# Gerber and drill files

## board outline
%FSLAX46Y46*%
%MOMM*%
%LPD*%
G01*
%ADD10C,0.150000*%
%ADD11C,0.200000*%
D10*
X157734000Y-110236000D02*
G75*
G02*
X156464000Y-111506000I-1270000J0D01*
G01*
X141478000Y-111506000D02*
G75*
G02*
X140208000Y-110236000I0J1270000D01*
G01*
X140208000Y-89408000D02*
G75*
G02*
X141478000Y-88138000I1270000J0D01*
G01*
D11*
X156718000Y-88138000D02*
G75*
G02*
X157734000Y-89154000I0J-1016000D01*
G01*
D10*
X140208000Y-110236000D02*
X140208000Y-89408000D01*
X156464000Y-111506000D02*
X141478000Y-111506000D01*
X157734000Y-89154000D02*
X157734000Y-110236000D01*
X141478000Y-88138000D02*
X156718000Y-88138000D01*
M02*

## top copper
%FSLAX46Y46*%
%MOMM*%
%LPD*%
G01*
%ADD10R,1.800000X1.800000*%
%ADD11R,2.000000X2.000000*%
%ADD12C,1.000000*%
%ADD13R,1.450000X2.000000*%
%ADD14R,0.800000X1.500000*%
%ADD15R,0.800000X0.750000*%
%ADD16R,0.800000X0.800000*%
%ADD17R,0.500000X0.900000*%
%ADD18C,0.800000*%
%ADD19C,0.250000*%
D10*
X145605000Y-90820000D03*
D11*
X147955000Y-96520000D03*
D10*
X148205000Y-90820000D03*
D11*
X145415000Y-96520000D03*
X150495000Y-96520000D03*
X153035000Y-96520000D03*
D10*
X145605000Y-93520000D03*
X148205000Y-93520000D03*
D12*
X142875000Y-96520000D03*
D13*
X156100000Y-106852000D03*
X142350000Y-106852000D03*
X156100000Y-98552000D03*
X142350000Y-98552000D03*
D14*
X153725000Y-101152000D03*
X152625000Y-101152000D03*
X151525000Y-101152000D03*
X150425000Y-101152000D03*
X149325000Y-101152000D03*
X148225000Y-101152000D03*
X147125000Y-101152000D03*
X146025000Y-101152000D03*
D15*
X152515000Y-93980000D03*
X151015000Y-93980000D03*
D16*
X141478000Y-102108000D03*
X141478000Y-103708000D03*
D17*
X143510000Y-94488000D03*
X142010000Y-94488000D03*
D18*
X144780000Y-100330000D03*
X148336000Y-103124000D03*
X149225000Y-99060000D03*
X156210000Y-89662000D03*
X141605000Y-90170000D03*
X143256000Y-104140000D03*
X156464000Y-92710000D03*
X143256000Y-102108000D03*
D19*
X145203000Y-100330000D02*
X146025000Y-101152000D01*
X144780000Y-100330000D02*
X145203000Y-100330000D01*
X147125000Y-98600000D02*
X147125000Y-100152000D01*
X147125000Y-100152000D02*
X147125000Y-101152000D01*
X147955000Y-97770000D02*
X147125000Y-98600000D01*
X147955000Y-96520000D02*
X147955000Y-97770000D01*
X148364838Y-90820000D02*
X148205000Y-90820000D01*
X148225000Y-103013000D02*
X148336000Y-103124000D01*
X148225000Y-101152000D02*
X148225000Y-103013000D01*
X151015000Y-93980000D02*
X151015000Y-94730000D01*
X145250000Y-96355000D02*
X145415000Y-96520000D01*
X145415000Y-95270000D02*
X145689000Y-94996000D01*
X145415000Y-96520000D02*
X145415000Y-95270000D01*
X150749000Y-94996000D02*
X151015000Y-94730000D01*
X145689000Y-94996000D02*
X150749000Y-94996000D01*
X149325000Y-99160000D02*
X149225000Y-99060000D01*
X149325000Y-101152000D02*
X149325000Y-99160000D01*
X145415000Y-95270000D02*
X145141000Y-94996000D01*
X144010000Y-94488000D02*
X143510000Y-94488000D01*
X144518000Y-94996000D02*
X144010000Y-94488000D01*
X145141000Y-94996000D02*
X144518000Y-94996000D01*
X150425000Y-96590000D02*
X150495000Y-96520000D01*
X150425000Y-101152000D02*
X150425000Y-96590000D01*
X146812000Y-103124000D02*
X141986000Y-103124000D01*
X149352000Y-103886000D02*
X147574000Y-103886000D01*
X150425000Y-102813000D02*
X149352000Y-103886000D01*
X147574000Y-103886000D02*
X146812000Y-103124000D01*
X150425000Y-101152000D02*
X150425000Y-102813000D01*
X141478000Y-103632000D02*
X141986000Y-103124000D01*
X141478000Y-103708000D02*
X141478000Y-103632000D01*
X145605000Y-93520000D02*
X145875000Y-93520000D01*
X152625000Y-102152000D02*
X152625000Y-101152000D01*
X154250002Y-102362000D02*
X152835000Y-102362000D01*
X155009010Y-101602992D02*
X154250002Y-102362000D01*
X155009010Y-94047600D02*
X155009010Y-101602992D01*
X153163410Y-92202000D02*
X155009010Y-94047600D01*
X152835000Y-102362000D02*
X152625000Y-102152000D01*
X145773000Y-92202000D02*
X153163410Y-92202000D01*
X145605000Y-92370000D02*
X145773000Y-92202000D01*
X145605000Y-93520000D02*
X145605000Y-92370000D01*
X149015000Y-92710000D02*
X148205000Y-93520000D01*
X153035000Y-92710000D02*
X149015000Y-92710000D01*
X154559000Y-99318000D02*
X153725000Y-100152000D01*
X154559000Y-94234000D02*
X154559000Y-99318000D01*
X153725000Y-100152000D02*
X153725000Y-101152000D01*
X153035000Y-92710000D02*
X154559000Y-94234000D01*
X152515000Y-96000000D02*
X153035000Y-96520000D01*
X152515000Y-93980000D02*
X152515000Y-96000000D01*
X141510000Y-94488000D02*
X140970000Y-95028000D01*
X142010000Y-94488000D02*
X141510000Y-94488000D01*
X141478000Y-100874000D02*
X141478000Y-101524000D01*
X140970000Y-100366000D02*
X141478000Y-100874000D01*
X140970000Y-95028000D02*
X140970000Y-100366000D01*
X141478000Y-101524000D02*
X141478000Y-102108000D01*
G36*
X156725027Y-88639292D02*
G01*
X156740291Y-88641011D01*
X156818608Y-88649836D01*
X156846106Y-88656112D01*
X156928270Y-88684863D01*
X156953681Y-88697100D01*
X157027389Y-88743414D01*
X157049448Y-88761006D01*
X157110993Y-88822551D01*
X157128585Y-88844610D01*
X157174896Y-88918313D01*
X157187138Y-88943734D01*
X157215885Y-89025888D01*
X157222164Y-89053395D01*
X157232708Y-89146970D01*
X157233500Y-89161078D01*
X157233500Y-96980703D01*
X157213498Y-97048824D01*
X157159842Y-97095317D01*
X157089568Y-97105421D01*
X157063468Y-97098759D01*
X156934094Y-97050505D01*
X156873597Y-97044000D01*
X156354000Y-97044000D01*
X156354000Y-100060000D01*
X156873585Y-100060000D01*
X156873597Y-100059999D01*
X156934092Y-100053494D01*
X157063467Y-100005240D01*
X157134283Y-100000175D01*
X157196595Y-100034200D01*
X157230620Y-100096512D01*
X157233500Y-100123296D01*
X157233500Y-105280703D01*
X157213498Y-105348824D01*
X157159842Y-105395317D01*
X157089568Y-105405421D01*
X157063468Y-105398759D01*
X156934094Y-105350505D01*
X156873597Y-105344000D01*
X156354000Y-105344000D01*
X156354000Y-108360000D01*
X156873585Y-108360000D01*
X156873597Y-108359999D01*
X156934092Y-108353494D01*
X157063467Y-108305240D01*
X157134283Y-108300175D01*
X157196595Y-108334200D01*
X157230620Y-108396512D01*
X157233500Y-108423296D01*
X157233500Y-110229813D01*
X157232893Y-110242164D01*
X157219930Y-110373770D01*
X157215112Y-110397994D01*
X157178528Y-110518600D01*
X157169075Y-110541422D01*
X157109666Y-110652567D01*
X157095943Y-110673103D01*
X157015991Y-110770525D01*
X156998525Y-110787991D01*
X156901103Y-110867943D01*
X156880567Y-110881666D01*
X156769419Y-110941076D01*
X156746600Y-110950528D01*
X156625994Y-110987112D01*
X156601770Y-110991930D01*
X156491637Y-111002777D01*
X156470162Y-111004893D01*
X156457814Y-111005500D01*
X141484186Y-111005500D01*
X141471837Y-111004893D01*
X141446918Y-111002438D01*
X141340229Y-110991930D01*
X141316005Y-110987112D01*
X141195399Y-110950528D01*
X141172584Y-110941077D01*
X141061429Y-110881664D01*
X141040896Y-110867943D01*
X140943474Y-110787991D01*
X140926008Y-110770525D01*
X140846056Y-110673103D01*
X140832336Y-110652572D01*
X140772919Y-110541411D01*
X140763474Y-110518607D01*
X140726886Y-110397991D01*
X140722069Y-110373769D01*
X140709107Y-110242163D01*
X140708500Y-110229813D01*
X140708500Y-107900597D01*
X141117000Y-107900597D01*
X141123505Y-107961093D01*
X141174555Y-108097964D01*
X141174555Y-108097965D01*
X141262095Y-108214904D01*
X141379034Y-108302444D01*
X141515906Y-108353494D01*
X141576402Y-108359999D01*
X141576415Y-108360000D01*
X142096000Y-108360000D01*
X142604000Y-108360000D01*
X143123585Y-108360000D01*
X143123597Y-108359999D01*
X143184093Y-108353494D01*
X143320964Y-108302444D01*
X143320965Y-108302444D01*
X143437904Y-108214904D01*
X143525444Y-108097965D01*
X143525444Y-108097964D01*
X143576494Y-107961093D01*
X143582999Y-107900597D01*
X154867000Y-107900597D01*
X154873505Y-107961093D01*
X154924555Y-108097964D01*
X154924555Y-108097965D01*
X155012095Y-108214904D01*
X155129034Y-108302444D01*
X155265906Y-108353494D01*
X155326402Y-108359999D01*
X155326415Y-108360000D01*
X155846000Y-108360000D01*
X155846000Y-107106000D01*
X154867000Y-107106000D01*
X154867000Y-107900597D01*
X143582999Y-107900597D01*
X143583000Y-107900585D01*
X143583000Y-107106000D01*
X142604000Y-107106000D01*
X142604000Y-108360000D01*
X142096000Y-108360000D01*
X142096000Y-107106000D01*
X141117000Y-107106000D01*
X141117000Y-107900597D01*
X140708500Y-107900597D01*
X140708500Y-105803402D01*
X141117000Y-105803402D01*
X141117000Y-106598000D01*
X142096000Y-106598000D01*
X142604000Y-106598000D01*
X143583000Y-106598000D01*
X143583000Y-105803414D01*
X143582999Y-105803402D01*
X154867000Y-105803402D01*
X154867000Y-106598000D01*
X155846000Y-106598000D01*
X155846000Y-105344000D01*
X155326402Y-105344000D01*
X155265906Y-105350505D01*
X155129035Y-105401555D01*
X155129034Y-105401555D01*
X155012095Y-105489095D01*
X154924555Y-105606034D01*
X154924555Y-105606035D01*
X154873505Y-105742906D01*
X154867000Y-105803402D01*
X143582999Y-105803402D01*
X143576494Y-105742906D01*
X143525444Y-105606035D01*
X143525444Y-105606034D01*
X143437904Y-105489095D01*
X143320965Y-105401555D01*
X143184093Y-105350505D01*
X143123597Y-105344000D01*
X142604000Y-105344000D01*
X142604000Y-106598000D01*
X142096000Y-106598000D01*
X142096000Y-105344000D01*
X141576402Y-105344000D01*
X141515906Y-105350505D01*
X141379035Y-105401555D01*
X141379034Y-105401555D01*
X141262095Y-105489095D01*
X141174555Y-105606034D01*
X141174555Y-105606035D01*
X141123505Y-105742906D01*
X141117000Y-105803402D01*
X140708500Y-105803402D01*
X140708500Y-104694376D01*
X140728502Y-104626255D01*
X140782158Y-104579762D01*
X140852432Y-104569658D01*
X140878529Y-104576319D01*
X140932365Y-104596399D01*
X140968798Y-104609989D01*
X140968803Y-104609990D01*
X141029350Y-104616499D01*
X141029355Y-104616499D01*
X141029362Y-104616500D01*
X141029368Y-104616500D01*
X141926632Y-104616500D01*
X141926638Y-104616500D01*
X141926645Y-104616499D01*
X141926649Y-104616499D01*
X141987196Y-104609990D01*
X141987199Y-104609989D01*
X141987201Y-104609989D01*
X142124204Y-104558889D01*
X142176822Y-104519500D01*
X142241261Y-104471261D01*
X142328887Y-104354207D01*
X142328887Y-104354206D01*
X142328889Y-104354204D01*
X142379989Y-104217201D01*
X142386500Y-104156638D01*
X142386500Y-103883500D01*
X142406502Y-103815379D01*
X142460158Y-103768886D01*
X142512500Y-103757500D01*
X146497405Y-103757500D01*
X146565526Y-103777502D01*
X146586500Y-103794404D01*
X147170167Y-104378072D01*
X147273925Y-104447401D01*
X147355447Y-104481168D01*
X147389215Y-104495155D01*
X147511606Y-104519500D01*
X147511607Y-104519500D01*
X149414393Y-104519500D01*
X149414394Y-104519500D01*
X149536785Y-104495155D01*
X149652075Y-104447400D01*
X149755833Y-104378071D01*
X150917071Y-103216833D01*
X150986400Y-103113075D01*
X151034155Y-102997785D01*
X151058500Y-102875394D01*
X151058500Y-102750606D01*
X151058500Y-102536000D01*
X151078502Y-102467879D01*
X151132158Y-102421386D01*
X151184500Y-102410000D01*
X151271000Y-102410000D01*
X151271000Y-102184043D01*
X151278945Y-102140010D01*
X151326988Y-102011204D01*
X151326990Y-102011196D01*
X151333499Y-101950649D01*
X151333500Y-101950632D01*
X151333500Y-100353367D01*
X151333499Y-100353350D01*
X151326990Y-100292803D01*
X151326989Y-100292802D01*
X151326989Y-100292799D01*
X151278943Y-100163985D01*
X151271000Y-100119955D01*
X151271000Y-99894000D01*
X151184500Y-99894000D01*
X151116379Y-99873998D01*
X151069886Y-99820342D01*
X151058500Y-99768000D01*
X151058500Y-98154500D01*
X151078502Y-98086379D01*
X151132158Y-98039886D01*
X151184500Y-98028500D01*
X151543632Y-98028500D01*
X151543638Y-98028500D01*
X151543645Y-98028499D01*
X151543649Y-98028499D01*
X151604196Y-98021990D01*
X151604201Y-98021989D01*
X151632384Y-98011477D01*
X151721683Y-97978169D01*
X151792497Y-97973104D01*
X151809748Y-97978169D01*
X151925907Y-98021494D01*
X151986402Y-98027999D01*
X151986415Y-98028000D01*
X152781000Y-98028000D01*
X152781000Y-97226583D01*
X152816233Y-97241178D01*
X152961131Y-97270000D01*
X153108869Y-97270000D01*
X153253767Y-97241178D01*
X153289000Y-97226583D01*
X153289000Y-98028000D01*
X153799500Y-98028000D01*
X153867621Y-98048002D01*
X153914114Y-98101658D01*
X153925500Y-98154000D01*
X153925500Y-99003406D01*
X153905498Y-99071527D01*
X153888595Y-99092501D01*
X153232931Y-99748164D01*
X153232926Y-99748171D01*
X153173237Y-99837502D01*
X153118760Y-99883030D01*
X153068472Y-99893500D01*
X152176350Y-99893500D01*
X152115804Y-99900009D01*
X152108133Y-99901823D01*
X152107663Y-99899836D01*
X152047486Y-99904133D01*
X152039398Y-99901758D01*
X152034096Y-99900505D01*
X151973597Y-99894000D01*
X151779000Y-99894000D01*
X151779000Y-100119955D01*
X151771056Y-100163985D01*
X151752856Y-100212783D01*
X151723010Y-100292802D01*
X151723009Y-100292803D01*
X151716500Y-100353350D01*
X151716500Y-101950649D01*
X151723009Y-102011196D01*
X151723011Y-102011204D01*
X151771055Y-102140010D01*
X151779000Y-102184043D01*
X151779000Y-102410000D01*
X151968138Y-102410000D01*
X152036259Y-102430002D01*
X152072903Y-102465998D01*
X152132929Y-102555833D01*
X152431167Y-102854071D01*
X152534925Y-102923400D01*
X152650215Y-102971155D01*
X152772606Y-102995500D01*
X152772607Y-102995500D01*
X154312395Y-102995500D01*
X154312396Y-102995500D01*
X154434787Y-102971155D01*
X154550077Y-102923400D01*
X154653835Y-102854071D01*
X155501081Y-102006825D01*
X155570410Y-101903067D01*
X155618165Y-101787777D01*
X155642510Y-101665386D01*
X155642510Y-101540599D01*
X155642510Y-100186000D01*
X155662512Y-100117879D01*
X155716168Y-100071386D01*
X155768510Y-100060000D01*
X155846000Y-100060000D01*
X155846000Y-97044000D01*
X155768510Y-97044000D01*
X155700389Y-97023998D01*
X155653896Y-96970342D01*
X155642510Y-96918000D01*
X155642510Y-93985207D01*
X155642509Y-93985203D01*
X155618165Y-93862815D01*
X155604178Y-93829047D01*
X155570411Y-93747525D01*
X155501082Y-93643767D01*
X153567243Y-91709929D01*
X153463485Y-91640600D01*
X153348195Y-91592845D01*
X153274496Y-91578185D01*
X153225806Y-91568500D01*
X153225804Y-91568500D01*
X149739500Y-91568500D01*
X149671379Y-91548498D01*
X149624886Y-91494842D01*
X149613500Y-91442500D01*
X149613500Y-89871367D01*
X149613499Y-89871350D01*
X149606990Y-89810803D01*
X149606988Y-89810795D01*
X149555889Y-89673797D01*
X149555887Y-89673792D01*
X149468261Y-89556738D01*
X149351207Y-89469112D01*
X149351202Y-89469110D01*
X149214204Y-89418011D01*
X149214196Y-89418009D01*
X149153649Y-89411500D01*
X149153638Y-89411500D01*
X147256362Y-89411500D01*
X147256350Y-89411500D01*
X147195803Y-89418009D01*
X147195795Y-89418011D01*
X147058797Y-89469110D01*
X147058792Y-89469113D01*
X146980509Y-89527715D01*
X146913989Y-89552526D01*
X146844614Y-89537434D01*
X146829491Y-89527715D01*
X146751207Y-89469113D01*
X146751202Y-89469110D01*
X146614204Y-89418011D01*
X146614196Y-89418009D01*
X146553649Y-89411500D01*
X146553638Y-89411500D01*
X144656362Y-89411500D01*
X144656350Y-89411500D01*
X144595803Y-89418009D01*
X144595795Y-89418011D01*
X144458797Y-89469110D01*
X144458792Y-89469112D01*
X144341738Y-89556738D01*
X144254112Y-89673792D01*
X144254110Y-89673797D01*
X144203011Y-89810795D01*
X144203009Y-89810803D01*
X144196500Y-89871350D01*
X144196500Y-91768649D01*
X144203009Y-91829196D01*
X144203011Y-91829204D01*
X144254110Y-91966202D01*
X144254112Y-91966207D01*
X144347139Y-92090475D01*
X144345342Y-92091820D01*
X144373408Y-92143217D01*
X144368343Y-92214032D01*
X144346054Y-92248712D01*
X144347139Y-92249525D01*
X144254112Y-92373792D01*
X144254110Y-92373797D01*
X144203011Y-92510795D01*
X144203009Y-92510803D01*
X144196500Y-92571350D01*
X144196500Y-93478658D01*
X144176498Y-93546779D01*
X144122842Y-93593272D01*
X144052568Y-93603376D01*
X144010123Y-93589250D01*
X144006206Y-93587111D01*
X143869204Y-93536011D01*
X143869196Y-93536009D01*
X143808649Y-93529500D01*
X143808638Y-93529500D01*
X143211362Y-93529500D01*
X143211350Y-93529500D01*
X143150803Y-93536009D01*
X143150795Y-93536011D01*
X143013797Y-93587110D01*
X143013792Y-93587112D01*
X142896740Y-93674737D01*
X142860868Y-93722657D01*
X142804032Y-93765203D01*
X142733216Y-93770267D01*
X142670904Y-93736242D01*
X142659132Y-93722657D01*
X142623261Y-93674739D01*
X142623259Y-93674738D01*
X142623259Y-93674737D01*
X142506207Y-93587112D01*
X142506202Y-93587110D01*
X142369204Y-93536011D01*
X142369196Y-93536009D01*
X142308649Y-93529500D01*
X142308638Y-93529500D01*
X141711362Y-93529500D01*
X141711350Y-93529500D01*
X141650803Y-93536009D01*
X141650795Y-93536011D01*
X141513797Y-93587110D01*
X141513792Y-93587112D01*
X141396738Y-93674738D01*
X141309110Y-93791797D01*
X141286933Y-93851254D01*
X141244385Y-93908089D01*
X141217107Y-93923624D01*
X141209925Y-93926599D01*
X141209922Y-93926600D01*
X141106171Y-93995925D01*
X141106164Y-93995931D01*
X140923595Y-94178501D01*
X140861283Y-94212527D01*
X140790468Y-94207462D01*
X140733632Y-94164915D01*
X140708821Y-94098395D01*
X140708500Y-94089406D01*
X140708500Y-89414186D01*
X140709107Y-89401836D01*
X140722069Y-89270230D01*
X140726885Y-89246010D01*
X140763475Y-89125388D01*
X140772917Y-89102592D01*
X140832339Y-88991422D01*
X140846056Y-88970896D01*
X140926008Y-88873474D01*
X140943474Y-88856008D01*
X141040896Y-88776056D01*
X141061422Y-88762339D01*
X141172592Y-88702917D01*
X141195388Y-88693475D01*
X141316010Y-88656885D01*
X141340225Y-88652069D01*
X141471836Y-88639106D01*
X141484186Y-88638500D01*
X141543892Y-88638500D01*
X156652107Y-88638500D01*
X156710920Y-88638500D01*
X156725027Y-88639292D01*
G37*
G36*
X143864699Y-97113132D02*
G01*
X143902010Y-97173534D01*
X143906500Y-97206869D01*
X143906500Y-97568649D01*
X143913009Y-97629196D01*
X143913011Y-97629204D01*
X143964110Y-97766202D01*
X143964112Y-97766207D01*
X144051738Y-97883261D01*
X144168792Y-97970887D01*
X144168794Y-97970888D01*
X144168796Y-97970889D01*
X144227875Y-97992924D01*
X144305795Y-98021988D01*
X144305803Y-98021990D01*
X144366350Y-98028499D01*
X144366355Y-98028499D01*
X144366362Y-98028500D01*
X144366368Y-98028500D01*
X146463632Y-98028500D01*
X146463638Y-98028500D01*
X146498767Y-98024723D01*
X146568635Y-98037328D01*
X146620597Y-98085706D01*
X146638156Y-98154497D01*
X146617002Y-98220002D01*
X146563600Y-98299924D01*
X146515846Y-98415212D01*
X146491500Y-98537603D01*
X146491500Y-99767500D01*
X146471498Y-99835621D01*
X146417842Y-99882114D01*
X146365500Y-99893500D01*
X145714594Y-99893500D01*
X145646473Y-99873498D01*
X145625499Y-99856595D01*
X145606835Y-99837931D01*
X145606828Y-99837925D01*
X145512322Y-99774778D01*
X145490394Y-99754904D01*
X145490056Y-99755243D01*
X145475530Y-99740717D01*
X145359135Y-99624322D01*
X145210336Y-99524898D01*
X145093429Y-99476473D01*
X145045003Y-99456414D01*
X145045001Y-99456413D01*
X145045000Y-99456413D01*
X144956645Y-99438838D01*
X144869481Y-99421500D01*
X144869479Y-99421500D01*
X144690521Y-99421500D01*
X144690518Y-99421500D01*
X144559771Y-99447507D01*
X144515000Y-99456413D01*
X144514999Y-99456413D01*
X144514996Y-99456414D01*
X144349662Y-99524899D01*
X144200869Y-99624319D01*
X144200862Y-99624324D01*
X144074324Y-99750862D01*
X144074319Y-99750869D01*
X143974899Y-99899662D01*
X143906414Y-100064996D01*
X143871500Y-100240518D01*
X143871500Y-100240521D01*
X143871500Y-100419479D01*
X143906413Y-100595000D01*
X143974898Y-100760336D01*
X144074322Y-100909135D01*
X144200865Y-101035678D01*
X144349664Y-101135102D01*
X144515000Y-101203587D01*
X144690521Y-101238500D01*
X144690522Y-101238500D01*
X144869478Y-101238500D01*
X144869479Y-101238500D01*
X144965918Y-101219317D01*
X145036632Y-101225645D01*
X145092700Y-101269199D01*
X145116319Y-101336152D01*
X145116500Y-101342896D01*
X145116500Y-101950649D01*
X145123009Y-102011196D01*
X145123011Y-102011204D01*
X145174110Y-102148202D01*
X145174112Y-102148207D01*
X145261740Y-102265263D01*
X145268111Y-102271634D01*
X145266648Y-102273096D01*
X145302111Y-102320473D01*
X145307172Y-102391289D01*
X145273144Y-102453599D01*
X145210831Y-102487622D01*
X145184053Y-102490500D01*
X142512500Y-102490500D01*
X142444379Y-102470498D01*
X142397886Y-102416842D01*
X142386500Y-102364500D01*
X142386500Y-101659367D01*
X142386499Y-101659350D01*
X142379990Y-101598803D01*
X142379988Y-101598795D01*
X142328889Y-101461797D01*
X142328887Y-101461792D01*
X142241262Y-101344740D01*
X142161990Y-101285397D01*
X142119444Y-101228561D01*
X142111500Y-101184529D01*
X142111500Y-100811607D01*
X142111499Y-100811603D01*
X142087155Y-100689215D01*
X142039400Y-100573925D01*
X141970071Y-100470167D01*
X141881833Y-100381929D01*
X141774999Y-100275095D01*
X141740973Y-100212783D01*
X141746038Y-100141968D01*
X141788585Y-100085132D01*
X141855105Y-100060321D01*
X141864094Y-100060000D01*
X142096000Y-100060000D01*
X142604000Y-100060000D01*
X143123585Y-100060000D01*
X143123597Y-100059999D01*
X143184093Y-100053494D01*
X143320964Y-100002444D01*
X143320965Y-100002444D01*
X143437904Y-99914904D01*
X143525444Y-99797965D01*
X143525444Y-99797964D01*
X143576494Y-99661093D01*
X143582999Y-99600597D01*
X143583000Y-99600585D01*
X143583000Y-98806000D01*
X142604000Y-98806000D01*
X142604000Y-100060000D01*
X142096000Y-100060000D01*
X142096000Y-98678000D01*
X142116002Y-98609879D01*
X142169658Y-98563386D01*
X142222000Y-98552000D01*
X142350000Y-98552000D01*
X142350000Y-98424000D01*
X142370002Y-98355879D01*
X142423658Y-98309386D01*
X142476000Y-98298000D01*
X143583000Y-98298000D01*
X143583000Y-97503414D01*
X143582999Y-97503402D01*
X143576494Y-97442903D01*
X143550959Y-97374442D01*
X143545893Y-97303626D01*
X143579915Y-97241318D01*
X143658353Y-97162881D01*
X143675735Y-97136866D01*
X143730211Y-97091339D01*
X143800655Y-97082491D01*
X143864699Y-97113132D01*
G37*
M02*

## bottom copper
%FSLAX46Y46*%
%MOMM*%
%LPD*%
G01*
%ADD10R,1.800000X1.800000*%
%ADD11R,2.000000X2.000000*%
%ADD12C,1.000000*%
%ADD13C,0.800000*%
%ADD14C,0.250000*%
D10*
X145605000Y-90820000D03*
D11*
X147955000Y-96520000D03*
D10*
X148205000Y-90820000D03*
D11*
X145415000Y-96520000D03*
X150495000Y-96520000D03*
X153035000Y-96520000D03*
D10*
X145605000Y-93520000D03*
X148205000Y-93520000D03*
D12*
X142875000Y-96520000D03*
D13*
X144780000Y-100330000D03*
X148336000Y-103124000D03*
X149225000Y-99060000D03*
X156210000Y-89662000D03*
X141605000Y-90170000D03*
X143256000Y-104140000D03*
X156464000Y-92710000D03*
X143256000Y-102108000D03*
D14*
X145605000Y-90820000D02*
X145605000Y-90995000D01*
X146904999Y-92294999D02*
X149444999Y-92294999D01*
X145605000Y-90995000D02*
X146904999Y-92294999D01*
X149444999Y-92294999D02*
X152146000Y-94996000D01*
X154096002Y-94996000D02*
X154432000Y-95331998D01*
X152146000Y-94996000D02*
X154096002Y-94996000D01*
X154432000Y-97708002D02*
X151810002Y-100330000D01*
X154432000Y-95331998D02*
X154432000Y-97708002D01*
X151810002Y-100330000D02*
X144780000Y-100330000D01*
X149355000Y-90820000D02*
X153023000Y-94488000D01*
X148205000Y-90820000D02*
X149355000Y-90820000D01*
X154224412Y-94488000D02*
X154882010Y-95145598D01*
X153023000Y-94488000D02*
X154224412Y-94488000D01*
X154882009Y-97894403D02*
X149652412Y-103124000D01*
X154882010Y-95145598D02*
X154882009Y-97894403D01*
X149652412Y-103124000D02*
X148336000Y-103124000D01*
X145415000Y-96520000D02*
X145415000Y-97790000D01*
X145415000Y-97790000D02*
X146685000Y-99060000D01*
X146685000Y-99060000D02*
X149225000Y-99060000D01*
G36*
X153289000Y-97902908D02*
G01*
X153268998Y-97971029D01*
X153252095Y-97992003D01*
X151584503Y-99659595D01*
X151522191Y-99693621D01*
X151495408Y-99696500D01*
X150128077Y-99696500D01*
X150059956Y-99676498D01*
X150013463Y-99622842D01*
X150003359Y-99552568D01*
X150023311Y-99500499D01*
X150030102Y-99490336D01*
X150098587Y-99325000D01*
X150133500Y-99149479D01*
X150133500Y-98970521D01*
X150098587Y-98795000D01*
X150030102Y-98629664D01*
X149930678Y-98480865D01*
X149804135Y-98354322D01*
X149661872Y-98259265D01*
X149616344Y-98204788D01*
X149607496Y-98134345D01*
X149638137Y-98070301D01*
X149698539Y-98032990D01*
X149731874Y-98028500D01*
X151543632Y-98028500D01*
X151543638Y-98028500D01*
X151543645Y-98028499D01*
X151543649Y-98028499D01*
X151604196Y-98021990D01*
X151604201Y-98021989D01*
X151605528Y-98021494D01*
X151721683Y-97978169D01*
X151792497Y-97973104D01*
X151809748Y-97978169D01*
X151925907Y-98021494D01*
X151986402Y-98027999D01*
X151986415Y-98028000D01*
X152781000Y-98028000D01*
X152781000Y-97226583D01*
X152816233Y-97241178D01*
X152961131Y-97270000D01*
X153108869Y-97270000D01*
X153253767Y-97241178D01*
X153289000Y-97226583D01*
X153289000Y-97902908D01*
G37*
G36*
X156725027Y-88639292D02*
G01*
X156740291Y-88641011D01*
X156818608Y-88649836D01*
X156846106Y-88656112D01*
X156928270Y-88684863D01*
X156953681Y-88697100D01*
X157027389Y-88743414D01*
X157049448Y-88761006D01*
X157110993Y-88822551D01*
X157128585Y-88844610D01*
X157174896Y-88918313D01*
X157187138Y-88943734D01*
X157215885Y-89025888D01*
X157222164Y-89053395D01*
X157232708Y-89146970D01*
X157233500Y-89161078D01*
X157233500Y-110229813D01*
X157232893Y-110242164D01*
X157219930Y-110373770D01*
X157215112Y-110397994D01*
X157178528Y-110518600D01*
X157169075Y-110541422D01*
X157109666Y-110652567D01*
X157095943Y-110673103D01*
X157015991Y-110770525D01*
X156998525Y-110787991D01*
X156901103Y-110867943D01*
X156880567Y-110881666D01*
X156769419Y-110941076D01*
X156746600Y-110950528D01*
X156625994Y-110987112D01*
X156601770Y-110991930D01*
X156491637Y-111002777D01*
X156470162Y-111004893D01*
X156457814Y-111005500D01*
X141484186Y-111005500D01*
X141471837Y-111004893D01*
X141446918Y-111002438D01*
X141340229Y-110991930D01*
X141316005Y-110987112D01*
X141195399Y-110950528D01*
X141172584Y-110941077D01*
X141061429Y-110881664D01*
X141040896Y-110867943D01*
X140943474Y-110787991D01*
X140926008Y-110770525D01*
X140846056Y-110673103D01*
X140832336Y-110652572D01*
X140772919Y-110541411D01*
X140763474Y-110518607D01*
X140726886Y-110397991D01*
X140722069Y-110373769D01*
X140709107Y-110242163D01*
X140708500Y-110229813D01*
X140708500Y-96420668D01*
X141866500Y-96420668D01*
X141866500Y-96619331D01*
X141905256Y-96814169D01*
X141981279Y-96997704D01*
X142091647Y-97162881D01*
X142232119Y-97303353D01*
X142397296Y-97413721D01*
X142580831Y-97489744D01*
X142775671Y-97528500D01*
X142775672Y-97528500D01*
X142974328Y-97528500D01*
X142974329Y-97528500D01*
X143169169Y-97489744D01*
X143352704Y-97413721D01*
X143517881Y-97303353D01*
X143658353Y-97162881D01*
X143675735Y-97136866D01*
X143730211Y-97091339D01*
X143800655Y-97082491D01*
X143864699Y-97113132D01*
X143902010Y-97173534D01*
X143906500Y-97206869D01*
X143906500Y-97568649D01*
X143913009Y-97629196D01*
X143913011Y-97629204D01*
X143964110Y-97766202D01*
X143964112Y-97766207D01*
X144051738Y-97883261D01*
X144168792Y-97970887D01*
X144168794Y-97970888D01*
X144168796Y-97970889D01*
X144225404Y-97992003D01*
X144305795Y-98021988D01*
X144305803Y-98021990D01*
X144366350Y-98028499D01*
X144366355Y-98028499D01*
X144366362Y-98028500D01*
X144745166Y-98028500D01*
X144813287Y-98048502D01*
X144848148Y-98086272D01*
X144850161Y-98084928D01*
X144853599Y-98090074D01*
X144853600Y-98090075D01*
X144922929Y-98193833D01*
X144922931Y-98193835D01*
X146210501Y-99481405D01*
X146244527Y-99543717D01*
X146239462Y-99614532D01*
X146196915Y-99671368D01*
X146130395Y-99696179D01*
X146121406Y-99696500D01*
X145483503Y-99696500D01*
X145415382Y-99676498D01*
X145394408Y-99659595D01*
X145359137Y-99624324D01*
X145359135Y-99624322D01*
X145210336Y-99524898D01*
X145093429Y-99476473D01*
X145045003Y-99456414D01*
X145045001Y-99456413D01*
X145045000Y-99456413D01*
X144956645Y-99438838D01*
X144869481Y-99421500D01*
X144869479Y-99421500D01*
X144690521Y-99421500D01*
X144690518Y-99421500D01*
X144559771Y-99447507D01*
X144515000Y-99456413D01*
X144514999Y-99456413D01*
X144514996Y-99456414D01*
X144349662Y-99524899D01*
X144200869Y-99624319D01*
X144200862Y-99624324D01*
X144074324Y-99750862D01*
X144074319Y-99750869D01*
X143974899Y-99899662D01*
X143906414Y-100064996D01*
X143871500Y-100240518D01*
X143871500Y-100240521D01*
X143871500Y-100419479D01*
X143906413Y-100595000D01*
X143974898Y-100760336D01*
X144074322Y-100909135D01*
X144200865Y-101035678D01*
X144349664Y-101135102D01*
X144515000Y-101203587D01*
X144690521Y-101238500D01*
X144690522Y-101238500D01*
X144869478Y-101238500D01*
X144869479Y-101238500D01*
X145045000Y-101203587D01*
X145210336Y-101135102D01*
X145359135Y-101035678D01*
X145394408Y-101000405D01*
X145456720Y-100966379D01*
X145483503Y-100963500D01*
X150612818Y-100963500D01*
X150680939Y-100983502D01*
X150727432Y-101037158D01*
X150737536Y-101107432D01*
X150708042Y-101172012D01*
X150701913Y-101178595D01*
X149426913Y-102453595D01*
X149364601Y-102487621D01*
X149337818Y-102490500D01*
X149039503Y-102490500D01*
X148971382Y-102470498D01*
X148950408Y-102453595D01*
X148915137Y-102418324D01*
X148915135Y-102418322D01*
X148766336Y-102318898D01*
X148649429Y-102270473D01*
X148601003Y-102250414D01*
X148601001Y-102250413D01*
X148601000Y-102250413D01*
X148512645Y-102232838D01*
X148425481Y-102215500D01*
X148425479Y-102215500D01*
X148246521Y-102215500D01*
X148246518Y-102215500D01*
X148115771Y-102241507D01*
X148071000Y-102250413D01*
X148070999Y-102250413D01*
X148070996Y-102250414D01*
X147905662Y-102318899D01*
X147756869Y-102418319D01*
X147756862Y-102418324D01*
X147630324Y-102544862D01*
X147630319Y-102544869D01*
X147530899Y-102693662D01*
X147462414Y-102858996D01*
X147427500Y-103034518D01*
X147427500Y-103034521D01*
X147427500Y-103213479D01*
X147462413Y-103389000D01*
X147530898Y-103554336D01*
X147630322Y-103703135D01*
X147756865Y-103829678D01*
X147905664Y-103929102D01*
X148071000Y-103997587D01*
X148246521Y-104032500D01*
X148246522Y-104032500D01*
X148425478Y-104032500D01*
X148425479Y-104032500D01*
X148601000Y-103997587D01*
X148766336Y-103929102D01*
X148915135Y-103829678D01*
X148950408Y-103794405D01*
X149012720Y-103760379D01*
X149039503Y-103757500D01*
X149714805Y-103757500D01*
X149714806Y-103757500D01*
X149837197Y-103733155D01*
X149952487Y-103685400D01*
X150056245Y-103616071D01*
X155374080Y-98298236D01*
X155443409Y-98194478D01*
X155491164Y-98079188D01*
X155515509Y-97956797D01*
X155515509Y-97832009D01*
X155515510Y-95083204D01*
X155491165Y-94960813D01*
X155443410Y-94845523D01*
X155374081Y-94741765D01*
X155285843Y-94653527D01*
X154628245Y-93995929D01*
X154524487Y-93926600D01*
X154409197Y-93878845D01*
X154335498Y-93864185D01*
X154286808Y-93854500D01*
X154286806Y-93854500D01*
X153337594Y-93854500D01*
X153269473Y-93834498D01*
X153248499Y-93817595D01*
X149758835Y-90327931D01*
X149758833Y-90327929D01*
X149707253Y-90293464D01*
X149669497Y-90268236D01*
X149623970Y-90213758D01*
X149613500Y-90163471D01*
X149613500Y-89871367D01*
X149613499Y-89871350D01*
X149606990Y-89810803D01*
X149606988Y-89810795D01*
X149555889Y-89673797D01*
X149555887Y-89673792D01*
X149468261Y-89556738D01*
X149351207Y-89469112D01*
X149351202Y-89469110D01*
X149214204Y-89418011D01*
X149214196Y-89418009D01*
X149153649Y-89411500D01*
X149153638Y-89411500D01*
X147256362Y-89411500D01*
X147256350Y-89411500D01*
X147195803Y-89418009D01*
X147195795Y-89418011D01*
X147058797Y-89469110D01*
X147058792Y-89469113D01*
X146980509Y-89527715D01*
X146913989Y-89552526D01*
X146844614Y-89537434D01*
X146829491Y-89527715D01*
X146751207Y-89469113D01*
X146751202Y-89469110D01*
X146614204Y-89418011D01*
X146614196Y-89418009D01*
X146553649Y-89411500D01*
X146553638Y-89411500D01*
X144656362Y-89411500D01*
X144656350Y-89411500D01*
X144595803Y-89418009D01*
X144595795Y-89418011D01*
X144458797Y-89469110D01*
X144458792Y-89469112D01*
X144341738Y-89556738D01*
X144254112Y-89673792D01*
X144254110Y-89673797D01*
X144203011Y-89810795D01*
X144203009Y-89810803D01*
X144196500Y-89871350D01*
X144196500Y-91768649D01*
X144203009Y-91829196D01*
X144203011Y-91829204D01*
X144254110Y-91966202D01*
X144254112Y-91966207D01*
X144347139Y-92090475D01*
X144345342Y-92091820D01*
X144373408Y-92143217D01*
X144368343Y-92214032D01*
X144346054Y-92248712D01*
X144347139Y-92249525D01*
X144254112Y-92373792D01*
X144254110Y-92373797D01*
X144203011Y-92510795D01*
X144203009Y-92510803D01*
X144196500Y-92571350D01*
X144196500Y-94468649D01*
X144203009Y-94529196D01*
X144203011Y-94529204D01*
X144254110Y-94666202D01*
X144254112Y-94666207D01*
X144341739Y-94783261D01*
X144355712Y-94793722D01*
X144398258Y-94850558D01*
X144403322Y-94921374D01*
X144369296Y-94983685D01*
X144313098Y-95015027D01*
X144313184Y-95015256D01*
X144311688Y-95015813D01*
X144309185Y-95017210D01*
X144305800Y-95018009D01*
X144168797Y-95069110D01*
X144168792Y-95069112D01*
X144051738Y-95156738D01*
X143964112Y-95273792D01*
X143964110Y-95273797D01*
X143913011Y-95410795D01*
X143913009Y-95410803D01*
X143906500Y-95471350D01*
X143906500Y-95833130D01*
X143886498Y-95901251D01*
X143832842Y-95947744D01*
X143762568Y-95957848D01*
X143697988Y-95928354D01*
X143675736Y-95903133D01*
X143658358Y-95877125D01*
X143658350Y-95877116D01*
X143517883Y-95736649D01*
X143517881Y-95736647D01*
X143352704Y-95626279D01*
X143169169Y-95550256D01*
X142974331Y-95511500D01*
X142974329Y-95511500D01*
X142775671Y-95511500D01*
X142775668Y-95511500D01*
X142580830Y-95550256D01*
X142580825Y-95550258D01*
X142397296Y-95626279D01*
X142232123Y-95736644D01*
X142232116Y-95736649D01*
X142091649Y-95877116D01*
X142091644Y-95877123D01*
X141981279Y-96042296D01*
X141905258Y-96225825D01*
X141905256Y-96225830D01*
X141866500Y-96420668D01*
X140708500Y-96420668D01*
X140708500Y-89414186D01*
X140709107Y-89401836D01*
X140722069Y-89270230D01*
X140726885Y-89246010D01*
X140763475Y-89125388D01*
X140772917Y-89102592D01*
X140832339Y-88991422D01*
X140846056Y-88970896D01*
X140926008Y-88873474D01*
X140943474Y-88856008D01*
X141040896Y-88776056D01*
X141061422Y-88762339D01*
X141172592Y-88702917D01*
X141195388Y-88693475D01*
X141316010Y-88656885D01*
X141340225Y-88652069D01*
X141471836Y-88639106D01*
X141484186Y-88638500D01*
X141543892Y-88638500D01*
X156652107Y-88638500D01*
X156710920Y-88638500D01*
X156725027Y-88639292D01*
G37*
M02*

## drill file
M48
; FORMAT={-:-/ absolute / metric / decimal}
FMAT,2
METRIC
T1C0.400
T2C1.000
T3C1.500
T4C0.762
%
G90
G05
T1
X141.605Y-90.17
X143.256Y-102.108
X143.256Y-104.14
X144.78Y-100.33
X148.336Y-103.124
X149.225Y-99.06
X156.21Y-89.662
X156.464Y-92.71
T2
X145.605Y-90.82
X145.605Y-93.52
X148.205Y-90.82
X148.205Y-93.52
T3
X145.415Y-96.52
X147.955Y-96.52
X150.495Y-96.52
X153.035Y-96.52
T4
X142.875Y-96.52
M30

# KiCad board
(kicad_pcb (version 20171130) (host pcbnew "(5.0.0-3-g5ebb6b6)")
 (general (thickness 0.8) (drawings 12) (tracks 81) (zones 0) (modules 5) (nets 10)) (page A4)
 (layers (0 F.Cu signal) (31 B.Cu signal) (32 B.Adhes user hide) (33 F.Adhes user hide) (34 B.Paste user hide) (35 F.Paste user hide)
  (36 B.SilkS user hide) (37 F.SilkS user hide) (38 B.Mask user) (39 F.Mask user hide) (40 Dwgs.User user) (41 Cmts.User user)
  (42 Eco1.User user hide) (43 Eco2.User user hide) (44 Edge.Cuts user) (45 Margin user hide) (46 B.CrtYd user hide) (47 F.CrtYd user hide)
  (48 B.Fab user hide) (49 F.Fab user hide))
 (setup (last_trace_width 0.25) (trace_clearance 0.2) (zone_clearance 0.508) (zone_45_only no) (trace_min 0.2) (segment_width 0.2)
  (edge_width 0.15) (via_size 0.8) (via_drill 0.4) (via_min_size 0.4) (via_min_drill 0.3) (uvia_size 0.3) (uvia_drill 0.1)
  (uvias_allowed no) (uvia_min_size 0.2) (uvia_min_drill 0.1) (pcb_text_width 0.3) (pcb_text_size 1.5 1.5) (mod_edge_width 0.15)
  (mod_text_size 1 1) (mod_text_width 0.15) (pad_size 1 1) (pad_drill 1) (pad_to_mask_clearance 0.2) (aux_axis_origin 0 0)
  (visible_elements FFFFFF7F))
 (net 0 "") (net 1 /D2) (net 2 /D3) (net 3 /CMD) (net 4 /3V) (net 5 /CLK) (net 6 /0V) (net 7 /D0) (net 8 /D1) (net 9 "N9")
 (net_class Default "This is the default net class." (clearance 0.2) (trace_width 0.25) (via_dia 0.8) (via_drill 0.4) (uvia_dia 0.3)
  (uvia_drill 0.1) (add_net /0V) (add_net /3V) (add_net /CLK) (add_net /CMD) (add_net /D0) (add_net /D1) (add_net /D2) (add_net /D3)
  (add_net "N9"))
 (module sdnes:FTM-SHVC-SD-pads (layer F.Cu) (at 147.955 96.52)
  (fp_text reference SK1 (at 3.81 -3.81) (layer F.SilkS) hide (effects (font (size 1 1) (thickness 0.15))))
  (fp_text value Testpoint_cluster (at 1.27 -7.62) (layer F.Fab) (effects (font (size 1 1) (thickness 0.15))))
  (pad 1 thru_hole rect (at -2.35 -5.7) (size 1.8 1.8) (drill 1) (layers *.Cu *.Mask) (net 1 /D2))
  (pad 2 thru_hole rect (at 0 0) (size 2 2) (drill 1.5) (layers *.Cu *.Mask) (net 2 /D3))
  (pad 3 thru_hole rect (at 0.25 -5.7) (size 1.8 1.8) (drill 1) (layers *.Cu *.Mask) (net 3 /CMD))
  (pad 4 thru_hole rect (at -2.54 0) (size 2 2) (drill 1.5) (layers *.Cu *.Mask) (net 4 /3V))
  (pad 5 thru_hole rect (at 2.54 0) (size 2 2) (drill 1.5) (layers *.Cu *.Mask) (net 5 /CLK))
  (pad 6 thru_hole rect (at 5.08 0) (size 2 2) (drill 1.5) (layers *.Cu *.Mask) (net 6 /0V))
  (pad 7 thru_hole rect (at -2.35 -3) (size 1.8 1.8) (drill 1) (layers *.Cu *.Mask) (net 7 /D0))
  (pad 8 thru_hole rect (at 0.25 -3) (size 1.8 1.8) (drill 1) (layers *.Cu *.Mask) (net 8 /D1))
  (pad "" np_thru_hole circle (at -5.08 0) (size 1 1) (drill 0.762) (layers *.Cu *.Mask)))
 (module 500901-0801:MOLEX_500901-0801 (layer F.Cu) (at 149.225 101.152)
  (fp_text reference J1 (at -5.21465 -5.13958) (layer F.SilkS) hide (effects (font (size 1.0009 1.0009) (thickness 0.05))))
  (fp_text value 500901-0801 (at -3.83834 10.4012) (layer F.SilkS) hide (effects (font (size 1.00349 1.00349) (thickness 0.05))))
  (pad SH4 smd rect (at 6.875 5.7 90) (size 2 1.45) (layers F.Cu F.Paste F.Mask) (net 6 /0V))
  (pad SH3 smd rect (at -6.875 5.7 90) (size 2 1.45) (layers F.Cu F.Paste F.Mask) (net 6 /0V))
  (pad SH2 smd rect (at 6.875 -2.6 90) (size 2 1.45) (layers F.Cu F.Paste F.Mask) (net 6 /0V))
  (pad SH1 smd rect (at -6.875 -2.6 90) (size 2 1.45) (layers F.Cu F.Paste F.Mask) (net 6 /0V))
  (pad 8 smd rect (at 4.5 0 90) (size 1.5 0.8) (layers F.Cu F.Paste F.Mask) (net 8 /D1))
  (pad 7 smd rect (at 3.4 0 90) (size 1.5 0.8) (layers F.Cu F.Paste F.Mask) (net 7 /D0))
  (pad 6 smd rect (at 2.3 0 90) (size 1.5 0.8) (layers F.Cu F.Paste F.Mask) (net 6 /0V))
  (pad 5 smd rect (at 1.2 0 90) (size 1.5 0.8) (layers F.Cu F.Paste F.Mask) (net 5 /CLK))
  (pad 4 smd rect (at 0.1 0 90) (size 1.5 0.8) (layers F.Cu F.Paste F.Mask) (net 4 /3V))
  (pad 3 smd rect (at -1 0 90) (size 1.5 0.8) (layers F.Cu F.Paste F.Mask) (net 3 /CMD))
  (pad 2 smd rect (at -2.1 0 90) (size 1.5 0.8) (layers F.Cu F.Paste F.Mask) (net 2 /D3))
  (pad 1 smd rect (at -3.2 0 90) (size 1.5 0.8) (layers F.Cu F.Paste F.Mask) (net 1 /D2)))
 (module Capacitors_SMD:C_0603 (layer F.Cu) (at 151.765 93.98)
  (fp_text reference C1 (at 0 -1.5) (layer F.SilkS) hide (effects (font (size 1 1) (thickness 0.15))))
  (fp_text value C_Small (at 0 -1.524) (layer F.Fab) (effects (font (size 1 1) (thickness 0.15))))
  (pad 2 smd rect (at 0.75 0) (size 0.8 0.75) (layers F.Cu F.Paste F.Mask) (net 6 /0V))
  (pad 1 smd rect (at -0.75 0) (size 0.8 0.75) (layers F.Cu F.Paste F.Mask) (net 4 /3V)))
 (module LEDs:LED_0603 (layer F.Cu) (at 141.478 102.908 90)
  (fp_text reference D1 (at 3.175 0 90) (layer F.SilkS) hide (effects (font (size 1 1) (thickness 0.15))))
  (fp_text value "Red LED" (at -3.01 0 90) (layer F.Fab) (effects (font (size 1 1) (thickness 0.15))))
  (pad 2 smd rect (at 0.8 0 270) (size 0.8 0.8) (layers F.Cu F.Paste F.Mask) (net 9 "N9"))
  (pad 1 smd rect (at -0.8 0 270) (size 0.8 0.8) (layers F.Cu F.Paste F.Mask) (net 5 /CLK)))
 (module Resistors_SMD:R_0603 (layer F.Cu) (at 142.76 94.488 180)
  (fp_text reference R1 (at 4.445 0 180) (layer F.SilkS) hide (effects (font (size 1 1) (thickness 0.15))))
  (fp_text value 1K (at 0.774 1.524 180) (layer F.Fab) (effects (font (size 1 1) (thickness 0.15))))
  (pad 1 smd rect (at -0.75 0 180) (size 0.5 0.9) (layers F.Cu F.Paste F.Mask) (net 4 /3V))
  (pad 2 smd rect (at 0.75 0 180) (size 0.5 0.9) (layers F.Cu F.Paste F.Mask) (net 9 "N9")))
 (gr_arc (start 156.464 110.236) (end 156.464 111.506) (angle -90) (layer Edge.Cuts) (width 0.15))
 (gr_arc (start 141.478 110.236) (end 140.208 110.236) (angle -90) (layer Edge.Cuts) (width 0.15))
 (gr_arc (start 141.478 89.408) (end 141.478 88.138) (angle -90) (layer Edge.Cuts) (width 0.15))
 (gr_arc (start 156.718 89.154) (end 157.734 89.154) (angle -90) (layer Edge.Cuts) (width 0.2))
 (gr_line (start 140.208 110.236) (end 140.208 89.408) (layer Edge.Cuts) (width 0.15))
 (gr_line (start 156.464 111.506) (end 141.478 111.506) (layer Edge.Cuts) (width 0.15))
 (gr_line (start 157.734 89.154) (end 157.734 110.236) (layer Edge.Cuts) (width 0.15))
 (gr_line (start 141.478 88.138) (end 156.718 88.138) (layer Edge.Cuts) (width 0.15))
 (segment (start 145.605 90.82) (end 145.605 90.995) (width 0.25) (layer B.Cu) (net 1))
 (segment (start 146.904999 92.294999) (end 149.444999 92.294999) (width 0.25) (layer B.Cu) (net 1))
 (segment (start 145.605 90.995) (end 146.904999 92.294999) (width 0.25) (layer B.Cu) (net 1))
 (segment (start 149.444999 92.294999) (end 152.146 94.996) (width 0.25) (layer B.Cu) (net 1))
 (segment (start 154.096002 94.996) (end 154.432 95.331998) (width 0.25) (layer B.Cu) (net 1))
 (segment (start 152.146 94.996) (end 154.096002 94.996) (width 0.25) (layer B.Cu) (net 1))
 (segment (start 154.432 97.708002) (end 151.810002 100.33) (width 0.25) (layer B.Cu) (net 1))
 (segment (start 154.432 95.331998) (end 154.432 97.708002) (width 0.25) (layer B.Cu) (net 1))
 (via (at 144.78 100.33) (size 0.8) (drill 0.4) (layers F.Cu B.Cu) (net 1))
 (segment (start 151.810002 100.33) (end 144.78 100.33) (width 0.25) (layer B.Cu) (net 1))
 (segment (start 145.203 100.33) (end 146.025 101.152) (width 0.25) (layer F.Cu) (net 1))
 (segment (start 144.78 100.33) (end 145.203 100.33) (width 0.25) (layer F.Cu) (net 1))
 (segment (start 147.125 98.6) (end 147.125 100.152) (width 0.25) (layer F.Cu) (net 2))
 (segment (start 147.125 100.152) (end 147.125 101.152) (width 0.25) (layer F.Cu) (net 2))
 (segment (start 147.955 97.77) (end 147.125 98.6) (width 0.25) (layer F.Cu) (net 2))
 (segment (start 147.955 96.52) (end 147.955 97.77) (width 0.25) (layer F.Cu) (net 2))
 (segment (start 148.364838 90.82) (end 148.205 90.82) (width 0.25) (layer F.Cu) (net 3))
 (segment (start 149.355 90.82) (end 153.023 94.488) (width 0.25) (layer B.Cu) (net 3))
 (segment (start 148.205 90.82) (end 149.355 90.82) (width 0.25) (layer B.Cu) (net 3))
 (segment (start 154.224412 94.488) (end 154.88201 95.145598) (width 0.25) (layer B.Cu) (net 3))
 (segment (start 153.023 94.488) (end 154.224412 94.488) (width 0.25) (layer B.Cu) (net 3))
 (segment (start 154.882009 97.894403) (end 149.652412 103.124) (width 0.25) (layer B.Cu) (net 3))
 (segment (start 154.88201 95.145598) (end 154.882009 97.894403) (width 0.25) (layer B.Cu) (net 3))
 (segment (start 149.652412 103.124) (end 148.336 103.124) (width 0.25) (layer B.Cu) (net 3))
 (via (at 148.336 103.124) (size 0.8) (drill 0.4) (layers F.Cu B.Cu) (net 3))
 (segment (start 148.225 103.013) (end 148.336 103.124) (width 0.25) (layer F.Cu) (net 3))
 (segment (start 148.225 101.152) (end 148.225 103.013) (width 0.25) (layer F.Cu) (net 3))
 (segment (start 145.415 96.52) (end 145.415 97.79) (width 0.25) (layer B.Cu) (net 4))
 (segment (start 145.415 97.79) (end 146.685 99.06) (width 0.25) (layer B.Cu) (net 4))
 (segment (start 146.685 99.06) (end 149.225 99.06) (width 0.25) (layer B.Cu) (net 4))
 (via (at 149.225 99.06) (size 0.8) (drill 0.4) (layers F.Cu B.Cu) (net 4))
 (segment (start 151.015 93.98) (end 151.015 94.73) (width 0.25) (layer F.Cu) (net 4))
 (segment (start 145.25 96.355) (end 145.415 96.52) (width 0.25) (layer F.Cu) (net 4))
 (segment (start 145.415 95.27) (end 145.689 94.996) (width 0.25) (layer F.Cu) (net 4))
 (segment (start 145.415 96.52) (end 145.415 95.27) (width 0.25) (layer F.Cu) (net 4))
 (segment (start 150.749 94.996) (end 151.015 94.73) (width 0.25) (layer F.Cu) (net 4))
 (segment (start 145.689 94.996) (end 150.749 94.996) (width 0.25) (layer F.Cu) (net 4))
 (segment (start 149.325 99.16) (end 149.225 99.06) (width 0.25) (layer F.Cu) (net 4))
 (segment (start 149.325 101.152) (end 149.325 99.16) (width 0.25) (layer F.Cu) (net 4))
 (segment (start 145.415 95.27) (end 145.141 94.996) (width 0.25) (layer F.Cu) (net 4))
 (segment (start 144.01 94.488) (end 143.51 94.488) (width 0.25) (layer F.Cu) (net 4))
 (segment (start 144.518 94.996) (end 144.01 94.488) (width 0.25) (layer F.Cu) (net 4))
 (segment (start 145.141 94.996) (end 144.518 94.996) (width 0.25) (layer F.Cu) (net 4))
 (segment (start 150.425 96.59) (end 150.495 96.52) (width 0.25) (layer F.Cu) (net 5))
 (segment (start 150.425 101.152) (end 150.425 96.59) (width 0.25) (layer F.Cu) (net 5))
 (segment (start 146.812 103.124) (end 141.986 103.124) (width 0.25) (layer F.Cu) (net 5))
 (segment (start 149.352 103.886) (end 147.574 103.886) (width 0.25) (layer F.Cu) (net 5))
 (segment (start 150.425 102.813) (end 149.352 103.886) (width 0.25) (layer F.Cu) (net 5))
 (segment (start 147.574 103.886) (end 146.812 103.124) (width 0.25) (layer F.Cu) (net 5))
 (segment (start 150.425 101.152) (end 150.425 102.813) (width 0.25) (layer F.Cu) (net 5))
 (segment (start 141.478 103.632) (end 141.986 103.124) (width 0.25) (layer F.Cu) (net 5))
 (segment (start 141.478 103.708) (end 141.478 103.632) (width 0.25) (layer F.Cu) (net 5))
 (segment (start 145.605 93.52) (end 145.875 93.52) (width 0.25) (layer F.Cu) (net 7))
 (segment (start 152.625 102.152) (end 152.625 101.152) (width 0.25) (layer F.Cu) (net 7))
 (segment (start 154.250002 102.362) (end 152.835 102.362) (width 0.25) (layer F.Cu) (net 7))
 (segment (start 155.00901 101.602992) (end 154.250002 102.362) (width 0.25) (layer F.Cu) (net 7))
 (segment (start 155.00901 94.0476) (end 155.00901 101.602992) (width 0.25) (layer F.Cu) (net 7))
 (segment (start 153.16341 92.202) (end 155.00901 94.0476) (width 0.25) (layer F.Cu) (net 7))
 (segment (start 152.835 102.362) (end 152.625 102.152) (width 0.25) (layer F.Cu) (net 7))
 (segment (start 145.773 92.202) (end 153.16341 92.202) (width 0.25) (layer F.Cu) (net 7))
 (segment (start 145.605 92.37) (end 145.773 92.202) (width 0.25) (layer F.Cu) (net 7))
 (segment (start 145.605 93.52) (end 145.605 92.37) (width 0.25) (layer F.Cu) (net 7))
 (segment (start 149.015 92.71) (end 148.205 93.52) (width 0.25) (layer F.Cu) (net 8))
 (segment (start 153.035 92.71) (end 149.015 92.71) (width 0.25) (layer F.Cu) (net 8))
 (segment (start 154.559 99.318) (end 153.725 100.152) (width 0.25) (layer F.Cu) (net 8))
 (segment (start 154.559 94.234) (end 154.559 99.318) (width 0.25) (layer F.Cu) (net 8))
 (segment (start 153.725 100.152) (end 153.725 101.152) (width 0.25) (layer F.Cu) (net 8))
 (segment (start 153.035 92.71) (end 154.559 94.234) (width 0.25) (layer F.Cu) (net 8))
 (segment (start 152.515 96) (end 153.035 96.52) (width 0.25) (layer F.Cu) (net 6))
 (via (at 156.21 89.662) (size 0.8) (drill 0.4) (layers F.Cu B.Cu) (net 6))
 (via (at 141.605 90.17) (size 0.8) (drill 0.4) (layers F.Cu B.Cu) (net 6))
 (via (at 143.256 104.14) (size 0.8) (drill 0.4) (layers F.Cu B.Cu) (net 6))
 (via (at 156.464 92.71) (size 0.8) (drill 0.4) (layers F.Cu B.Cu) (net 6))
 (segment (start 152.515 93.98) (end 152.515 96) (width 0.25) (layer F.Cu) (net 6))
 (via (at 143.256 102.108) (size 0.8) (drill 0.4) (layers F.Cu B.Cu) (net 6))
 (segment (start 141.51 94.488) (end 140.97 95.028) (width 0.25) (layer F.Cu) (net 9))
 (segment (start 142.01 94.488) (end 141.51 94.488) (width 0.25) (layer F.Cu) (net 9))
 (segment (start 141.478 100.874) (end 141.478 101.524) (width 0.25) (layer F.Cu) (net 9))
 (segment (start 140.97 100.366) (end 141.478 100.874) (width 0.25) (layer F.Cu) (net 9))
 (segment (start 140.97 95.028) (end 140.97 100.366) (width 0.25) (layer F.Cu) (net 9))
 (segment (start 141.478 101.524) (end 141.478 102.108) (width 0.25) (layer F.Cu) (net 9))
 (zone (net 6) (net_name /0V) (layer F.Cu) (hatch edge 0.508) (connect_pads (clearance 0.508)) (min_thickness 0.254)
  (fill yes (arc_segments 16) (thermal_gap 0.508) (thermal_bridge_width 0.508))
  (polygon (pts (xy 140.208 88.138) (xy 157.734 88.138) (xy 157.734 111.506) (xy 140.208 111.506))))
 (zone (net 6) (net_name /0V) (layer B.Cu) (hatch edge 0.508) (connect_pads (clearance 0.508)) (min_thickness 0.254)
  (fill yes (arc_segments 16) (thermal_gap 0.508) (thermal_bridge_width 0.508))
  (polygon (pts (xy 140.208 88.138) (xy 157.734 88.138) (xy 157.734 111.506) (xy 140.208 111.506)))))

